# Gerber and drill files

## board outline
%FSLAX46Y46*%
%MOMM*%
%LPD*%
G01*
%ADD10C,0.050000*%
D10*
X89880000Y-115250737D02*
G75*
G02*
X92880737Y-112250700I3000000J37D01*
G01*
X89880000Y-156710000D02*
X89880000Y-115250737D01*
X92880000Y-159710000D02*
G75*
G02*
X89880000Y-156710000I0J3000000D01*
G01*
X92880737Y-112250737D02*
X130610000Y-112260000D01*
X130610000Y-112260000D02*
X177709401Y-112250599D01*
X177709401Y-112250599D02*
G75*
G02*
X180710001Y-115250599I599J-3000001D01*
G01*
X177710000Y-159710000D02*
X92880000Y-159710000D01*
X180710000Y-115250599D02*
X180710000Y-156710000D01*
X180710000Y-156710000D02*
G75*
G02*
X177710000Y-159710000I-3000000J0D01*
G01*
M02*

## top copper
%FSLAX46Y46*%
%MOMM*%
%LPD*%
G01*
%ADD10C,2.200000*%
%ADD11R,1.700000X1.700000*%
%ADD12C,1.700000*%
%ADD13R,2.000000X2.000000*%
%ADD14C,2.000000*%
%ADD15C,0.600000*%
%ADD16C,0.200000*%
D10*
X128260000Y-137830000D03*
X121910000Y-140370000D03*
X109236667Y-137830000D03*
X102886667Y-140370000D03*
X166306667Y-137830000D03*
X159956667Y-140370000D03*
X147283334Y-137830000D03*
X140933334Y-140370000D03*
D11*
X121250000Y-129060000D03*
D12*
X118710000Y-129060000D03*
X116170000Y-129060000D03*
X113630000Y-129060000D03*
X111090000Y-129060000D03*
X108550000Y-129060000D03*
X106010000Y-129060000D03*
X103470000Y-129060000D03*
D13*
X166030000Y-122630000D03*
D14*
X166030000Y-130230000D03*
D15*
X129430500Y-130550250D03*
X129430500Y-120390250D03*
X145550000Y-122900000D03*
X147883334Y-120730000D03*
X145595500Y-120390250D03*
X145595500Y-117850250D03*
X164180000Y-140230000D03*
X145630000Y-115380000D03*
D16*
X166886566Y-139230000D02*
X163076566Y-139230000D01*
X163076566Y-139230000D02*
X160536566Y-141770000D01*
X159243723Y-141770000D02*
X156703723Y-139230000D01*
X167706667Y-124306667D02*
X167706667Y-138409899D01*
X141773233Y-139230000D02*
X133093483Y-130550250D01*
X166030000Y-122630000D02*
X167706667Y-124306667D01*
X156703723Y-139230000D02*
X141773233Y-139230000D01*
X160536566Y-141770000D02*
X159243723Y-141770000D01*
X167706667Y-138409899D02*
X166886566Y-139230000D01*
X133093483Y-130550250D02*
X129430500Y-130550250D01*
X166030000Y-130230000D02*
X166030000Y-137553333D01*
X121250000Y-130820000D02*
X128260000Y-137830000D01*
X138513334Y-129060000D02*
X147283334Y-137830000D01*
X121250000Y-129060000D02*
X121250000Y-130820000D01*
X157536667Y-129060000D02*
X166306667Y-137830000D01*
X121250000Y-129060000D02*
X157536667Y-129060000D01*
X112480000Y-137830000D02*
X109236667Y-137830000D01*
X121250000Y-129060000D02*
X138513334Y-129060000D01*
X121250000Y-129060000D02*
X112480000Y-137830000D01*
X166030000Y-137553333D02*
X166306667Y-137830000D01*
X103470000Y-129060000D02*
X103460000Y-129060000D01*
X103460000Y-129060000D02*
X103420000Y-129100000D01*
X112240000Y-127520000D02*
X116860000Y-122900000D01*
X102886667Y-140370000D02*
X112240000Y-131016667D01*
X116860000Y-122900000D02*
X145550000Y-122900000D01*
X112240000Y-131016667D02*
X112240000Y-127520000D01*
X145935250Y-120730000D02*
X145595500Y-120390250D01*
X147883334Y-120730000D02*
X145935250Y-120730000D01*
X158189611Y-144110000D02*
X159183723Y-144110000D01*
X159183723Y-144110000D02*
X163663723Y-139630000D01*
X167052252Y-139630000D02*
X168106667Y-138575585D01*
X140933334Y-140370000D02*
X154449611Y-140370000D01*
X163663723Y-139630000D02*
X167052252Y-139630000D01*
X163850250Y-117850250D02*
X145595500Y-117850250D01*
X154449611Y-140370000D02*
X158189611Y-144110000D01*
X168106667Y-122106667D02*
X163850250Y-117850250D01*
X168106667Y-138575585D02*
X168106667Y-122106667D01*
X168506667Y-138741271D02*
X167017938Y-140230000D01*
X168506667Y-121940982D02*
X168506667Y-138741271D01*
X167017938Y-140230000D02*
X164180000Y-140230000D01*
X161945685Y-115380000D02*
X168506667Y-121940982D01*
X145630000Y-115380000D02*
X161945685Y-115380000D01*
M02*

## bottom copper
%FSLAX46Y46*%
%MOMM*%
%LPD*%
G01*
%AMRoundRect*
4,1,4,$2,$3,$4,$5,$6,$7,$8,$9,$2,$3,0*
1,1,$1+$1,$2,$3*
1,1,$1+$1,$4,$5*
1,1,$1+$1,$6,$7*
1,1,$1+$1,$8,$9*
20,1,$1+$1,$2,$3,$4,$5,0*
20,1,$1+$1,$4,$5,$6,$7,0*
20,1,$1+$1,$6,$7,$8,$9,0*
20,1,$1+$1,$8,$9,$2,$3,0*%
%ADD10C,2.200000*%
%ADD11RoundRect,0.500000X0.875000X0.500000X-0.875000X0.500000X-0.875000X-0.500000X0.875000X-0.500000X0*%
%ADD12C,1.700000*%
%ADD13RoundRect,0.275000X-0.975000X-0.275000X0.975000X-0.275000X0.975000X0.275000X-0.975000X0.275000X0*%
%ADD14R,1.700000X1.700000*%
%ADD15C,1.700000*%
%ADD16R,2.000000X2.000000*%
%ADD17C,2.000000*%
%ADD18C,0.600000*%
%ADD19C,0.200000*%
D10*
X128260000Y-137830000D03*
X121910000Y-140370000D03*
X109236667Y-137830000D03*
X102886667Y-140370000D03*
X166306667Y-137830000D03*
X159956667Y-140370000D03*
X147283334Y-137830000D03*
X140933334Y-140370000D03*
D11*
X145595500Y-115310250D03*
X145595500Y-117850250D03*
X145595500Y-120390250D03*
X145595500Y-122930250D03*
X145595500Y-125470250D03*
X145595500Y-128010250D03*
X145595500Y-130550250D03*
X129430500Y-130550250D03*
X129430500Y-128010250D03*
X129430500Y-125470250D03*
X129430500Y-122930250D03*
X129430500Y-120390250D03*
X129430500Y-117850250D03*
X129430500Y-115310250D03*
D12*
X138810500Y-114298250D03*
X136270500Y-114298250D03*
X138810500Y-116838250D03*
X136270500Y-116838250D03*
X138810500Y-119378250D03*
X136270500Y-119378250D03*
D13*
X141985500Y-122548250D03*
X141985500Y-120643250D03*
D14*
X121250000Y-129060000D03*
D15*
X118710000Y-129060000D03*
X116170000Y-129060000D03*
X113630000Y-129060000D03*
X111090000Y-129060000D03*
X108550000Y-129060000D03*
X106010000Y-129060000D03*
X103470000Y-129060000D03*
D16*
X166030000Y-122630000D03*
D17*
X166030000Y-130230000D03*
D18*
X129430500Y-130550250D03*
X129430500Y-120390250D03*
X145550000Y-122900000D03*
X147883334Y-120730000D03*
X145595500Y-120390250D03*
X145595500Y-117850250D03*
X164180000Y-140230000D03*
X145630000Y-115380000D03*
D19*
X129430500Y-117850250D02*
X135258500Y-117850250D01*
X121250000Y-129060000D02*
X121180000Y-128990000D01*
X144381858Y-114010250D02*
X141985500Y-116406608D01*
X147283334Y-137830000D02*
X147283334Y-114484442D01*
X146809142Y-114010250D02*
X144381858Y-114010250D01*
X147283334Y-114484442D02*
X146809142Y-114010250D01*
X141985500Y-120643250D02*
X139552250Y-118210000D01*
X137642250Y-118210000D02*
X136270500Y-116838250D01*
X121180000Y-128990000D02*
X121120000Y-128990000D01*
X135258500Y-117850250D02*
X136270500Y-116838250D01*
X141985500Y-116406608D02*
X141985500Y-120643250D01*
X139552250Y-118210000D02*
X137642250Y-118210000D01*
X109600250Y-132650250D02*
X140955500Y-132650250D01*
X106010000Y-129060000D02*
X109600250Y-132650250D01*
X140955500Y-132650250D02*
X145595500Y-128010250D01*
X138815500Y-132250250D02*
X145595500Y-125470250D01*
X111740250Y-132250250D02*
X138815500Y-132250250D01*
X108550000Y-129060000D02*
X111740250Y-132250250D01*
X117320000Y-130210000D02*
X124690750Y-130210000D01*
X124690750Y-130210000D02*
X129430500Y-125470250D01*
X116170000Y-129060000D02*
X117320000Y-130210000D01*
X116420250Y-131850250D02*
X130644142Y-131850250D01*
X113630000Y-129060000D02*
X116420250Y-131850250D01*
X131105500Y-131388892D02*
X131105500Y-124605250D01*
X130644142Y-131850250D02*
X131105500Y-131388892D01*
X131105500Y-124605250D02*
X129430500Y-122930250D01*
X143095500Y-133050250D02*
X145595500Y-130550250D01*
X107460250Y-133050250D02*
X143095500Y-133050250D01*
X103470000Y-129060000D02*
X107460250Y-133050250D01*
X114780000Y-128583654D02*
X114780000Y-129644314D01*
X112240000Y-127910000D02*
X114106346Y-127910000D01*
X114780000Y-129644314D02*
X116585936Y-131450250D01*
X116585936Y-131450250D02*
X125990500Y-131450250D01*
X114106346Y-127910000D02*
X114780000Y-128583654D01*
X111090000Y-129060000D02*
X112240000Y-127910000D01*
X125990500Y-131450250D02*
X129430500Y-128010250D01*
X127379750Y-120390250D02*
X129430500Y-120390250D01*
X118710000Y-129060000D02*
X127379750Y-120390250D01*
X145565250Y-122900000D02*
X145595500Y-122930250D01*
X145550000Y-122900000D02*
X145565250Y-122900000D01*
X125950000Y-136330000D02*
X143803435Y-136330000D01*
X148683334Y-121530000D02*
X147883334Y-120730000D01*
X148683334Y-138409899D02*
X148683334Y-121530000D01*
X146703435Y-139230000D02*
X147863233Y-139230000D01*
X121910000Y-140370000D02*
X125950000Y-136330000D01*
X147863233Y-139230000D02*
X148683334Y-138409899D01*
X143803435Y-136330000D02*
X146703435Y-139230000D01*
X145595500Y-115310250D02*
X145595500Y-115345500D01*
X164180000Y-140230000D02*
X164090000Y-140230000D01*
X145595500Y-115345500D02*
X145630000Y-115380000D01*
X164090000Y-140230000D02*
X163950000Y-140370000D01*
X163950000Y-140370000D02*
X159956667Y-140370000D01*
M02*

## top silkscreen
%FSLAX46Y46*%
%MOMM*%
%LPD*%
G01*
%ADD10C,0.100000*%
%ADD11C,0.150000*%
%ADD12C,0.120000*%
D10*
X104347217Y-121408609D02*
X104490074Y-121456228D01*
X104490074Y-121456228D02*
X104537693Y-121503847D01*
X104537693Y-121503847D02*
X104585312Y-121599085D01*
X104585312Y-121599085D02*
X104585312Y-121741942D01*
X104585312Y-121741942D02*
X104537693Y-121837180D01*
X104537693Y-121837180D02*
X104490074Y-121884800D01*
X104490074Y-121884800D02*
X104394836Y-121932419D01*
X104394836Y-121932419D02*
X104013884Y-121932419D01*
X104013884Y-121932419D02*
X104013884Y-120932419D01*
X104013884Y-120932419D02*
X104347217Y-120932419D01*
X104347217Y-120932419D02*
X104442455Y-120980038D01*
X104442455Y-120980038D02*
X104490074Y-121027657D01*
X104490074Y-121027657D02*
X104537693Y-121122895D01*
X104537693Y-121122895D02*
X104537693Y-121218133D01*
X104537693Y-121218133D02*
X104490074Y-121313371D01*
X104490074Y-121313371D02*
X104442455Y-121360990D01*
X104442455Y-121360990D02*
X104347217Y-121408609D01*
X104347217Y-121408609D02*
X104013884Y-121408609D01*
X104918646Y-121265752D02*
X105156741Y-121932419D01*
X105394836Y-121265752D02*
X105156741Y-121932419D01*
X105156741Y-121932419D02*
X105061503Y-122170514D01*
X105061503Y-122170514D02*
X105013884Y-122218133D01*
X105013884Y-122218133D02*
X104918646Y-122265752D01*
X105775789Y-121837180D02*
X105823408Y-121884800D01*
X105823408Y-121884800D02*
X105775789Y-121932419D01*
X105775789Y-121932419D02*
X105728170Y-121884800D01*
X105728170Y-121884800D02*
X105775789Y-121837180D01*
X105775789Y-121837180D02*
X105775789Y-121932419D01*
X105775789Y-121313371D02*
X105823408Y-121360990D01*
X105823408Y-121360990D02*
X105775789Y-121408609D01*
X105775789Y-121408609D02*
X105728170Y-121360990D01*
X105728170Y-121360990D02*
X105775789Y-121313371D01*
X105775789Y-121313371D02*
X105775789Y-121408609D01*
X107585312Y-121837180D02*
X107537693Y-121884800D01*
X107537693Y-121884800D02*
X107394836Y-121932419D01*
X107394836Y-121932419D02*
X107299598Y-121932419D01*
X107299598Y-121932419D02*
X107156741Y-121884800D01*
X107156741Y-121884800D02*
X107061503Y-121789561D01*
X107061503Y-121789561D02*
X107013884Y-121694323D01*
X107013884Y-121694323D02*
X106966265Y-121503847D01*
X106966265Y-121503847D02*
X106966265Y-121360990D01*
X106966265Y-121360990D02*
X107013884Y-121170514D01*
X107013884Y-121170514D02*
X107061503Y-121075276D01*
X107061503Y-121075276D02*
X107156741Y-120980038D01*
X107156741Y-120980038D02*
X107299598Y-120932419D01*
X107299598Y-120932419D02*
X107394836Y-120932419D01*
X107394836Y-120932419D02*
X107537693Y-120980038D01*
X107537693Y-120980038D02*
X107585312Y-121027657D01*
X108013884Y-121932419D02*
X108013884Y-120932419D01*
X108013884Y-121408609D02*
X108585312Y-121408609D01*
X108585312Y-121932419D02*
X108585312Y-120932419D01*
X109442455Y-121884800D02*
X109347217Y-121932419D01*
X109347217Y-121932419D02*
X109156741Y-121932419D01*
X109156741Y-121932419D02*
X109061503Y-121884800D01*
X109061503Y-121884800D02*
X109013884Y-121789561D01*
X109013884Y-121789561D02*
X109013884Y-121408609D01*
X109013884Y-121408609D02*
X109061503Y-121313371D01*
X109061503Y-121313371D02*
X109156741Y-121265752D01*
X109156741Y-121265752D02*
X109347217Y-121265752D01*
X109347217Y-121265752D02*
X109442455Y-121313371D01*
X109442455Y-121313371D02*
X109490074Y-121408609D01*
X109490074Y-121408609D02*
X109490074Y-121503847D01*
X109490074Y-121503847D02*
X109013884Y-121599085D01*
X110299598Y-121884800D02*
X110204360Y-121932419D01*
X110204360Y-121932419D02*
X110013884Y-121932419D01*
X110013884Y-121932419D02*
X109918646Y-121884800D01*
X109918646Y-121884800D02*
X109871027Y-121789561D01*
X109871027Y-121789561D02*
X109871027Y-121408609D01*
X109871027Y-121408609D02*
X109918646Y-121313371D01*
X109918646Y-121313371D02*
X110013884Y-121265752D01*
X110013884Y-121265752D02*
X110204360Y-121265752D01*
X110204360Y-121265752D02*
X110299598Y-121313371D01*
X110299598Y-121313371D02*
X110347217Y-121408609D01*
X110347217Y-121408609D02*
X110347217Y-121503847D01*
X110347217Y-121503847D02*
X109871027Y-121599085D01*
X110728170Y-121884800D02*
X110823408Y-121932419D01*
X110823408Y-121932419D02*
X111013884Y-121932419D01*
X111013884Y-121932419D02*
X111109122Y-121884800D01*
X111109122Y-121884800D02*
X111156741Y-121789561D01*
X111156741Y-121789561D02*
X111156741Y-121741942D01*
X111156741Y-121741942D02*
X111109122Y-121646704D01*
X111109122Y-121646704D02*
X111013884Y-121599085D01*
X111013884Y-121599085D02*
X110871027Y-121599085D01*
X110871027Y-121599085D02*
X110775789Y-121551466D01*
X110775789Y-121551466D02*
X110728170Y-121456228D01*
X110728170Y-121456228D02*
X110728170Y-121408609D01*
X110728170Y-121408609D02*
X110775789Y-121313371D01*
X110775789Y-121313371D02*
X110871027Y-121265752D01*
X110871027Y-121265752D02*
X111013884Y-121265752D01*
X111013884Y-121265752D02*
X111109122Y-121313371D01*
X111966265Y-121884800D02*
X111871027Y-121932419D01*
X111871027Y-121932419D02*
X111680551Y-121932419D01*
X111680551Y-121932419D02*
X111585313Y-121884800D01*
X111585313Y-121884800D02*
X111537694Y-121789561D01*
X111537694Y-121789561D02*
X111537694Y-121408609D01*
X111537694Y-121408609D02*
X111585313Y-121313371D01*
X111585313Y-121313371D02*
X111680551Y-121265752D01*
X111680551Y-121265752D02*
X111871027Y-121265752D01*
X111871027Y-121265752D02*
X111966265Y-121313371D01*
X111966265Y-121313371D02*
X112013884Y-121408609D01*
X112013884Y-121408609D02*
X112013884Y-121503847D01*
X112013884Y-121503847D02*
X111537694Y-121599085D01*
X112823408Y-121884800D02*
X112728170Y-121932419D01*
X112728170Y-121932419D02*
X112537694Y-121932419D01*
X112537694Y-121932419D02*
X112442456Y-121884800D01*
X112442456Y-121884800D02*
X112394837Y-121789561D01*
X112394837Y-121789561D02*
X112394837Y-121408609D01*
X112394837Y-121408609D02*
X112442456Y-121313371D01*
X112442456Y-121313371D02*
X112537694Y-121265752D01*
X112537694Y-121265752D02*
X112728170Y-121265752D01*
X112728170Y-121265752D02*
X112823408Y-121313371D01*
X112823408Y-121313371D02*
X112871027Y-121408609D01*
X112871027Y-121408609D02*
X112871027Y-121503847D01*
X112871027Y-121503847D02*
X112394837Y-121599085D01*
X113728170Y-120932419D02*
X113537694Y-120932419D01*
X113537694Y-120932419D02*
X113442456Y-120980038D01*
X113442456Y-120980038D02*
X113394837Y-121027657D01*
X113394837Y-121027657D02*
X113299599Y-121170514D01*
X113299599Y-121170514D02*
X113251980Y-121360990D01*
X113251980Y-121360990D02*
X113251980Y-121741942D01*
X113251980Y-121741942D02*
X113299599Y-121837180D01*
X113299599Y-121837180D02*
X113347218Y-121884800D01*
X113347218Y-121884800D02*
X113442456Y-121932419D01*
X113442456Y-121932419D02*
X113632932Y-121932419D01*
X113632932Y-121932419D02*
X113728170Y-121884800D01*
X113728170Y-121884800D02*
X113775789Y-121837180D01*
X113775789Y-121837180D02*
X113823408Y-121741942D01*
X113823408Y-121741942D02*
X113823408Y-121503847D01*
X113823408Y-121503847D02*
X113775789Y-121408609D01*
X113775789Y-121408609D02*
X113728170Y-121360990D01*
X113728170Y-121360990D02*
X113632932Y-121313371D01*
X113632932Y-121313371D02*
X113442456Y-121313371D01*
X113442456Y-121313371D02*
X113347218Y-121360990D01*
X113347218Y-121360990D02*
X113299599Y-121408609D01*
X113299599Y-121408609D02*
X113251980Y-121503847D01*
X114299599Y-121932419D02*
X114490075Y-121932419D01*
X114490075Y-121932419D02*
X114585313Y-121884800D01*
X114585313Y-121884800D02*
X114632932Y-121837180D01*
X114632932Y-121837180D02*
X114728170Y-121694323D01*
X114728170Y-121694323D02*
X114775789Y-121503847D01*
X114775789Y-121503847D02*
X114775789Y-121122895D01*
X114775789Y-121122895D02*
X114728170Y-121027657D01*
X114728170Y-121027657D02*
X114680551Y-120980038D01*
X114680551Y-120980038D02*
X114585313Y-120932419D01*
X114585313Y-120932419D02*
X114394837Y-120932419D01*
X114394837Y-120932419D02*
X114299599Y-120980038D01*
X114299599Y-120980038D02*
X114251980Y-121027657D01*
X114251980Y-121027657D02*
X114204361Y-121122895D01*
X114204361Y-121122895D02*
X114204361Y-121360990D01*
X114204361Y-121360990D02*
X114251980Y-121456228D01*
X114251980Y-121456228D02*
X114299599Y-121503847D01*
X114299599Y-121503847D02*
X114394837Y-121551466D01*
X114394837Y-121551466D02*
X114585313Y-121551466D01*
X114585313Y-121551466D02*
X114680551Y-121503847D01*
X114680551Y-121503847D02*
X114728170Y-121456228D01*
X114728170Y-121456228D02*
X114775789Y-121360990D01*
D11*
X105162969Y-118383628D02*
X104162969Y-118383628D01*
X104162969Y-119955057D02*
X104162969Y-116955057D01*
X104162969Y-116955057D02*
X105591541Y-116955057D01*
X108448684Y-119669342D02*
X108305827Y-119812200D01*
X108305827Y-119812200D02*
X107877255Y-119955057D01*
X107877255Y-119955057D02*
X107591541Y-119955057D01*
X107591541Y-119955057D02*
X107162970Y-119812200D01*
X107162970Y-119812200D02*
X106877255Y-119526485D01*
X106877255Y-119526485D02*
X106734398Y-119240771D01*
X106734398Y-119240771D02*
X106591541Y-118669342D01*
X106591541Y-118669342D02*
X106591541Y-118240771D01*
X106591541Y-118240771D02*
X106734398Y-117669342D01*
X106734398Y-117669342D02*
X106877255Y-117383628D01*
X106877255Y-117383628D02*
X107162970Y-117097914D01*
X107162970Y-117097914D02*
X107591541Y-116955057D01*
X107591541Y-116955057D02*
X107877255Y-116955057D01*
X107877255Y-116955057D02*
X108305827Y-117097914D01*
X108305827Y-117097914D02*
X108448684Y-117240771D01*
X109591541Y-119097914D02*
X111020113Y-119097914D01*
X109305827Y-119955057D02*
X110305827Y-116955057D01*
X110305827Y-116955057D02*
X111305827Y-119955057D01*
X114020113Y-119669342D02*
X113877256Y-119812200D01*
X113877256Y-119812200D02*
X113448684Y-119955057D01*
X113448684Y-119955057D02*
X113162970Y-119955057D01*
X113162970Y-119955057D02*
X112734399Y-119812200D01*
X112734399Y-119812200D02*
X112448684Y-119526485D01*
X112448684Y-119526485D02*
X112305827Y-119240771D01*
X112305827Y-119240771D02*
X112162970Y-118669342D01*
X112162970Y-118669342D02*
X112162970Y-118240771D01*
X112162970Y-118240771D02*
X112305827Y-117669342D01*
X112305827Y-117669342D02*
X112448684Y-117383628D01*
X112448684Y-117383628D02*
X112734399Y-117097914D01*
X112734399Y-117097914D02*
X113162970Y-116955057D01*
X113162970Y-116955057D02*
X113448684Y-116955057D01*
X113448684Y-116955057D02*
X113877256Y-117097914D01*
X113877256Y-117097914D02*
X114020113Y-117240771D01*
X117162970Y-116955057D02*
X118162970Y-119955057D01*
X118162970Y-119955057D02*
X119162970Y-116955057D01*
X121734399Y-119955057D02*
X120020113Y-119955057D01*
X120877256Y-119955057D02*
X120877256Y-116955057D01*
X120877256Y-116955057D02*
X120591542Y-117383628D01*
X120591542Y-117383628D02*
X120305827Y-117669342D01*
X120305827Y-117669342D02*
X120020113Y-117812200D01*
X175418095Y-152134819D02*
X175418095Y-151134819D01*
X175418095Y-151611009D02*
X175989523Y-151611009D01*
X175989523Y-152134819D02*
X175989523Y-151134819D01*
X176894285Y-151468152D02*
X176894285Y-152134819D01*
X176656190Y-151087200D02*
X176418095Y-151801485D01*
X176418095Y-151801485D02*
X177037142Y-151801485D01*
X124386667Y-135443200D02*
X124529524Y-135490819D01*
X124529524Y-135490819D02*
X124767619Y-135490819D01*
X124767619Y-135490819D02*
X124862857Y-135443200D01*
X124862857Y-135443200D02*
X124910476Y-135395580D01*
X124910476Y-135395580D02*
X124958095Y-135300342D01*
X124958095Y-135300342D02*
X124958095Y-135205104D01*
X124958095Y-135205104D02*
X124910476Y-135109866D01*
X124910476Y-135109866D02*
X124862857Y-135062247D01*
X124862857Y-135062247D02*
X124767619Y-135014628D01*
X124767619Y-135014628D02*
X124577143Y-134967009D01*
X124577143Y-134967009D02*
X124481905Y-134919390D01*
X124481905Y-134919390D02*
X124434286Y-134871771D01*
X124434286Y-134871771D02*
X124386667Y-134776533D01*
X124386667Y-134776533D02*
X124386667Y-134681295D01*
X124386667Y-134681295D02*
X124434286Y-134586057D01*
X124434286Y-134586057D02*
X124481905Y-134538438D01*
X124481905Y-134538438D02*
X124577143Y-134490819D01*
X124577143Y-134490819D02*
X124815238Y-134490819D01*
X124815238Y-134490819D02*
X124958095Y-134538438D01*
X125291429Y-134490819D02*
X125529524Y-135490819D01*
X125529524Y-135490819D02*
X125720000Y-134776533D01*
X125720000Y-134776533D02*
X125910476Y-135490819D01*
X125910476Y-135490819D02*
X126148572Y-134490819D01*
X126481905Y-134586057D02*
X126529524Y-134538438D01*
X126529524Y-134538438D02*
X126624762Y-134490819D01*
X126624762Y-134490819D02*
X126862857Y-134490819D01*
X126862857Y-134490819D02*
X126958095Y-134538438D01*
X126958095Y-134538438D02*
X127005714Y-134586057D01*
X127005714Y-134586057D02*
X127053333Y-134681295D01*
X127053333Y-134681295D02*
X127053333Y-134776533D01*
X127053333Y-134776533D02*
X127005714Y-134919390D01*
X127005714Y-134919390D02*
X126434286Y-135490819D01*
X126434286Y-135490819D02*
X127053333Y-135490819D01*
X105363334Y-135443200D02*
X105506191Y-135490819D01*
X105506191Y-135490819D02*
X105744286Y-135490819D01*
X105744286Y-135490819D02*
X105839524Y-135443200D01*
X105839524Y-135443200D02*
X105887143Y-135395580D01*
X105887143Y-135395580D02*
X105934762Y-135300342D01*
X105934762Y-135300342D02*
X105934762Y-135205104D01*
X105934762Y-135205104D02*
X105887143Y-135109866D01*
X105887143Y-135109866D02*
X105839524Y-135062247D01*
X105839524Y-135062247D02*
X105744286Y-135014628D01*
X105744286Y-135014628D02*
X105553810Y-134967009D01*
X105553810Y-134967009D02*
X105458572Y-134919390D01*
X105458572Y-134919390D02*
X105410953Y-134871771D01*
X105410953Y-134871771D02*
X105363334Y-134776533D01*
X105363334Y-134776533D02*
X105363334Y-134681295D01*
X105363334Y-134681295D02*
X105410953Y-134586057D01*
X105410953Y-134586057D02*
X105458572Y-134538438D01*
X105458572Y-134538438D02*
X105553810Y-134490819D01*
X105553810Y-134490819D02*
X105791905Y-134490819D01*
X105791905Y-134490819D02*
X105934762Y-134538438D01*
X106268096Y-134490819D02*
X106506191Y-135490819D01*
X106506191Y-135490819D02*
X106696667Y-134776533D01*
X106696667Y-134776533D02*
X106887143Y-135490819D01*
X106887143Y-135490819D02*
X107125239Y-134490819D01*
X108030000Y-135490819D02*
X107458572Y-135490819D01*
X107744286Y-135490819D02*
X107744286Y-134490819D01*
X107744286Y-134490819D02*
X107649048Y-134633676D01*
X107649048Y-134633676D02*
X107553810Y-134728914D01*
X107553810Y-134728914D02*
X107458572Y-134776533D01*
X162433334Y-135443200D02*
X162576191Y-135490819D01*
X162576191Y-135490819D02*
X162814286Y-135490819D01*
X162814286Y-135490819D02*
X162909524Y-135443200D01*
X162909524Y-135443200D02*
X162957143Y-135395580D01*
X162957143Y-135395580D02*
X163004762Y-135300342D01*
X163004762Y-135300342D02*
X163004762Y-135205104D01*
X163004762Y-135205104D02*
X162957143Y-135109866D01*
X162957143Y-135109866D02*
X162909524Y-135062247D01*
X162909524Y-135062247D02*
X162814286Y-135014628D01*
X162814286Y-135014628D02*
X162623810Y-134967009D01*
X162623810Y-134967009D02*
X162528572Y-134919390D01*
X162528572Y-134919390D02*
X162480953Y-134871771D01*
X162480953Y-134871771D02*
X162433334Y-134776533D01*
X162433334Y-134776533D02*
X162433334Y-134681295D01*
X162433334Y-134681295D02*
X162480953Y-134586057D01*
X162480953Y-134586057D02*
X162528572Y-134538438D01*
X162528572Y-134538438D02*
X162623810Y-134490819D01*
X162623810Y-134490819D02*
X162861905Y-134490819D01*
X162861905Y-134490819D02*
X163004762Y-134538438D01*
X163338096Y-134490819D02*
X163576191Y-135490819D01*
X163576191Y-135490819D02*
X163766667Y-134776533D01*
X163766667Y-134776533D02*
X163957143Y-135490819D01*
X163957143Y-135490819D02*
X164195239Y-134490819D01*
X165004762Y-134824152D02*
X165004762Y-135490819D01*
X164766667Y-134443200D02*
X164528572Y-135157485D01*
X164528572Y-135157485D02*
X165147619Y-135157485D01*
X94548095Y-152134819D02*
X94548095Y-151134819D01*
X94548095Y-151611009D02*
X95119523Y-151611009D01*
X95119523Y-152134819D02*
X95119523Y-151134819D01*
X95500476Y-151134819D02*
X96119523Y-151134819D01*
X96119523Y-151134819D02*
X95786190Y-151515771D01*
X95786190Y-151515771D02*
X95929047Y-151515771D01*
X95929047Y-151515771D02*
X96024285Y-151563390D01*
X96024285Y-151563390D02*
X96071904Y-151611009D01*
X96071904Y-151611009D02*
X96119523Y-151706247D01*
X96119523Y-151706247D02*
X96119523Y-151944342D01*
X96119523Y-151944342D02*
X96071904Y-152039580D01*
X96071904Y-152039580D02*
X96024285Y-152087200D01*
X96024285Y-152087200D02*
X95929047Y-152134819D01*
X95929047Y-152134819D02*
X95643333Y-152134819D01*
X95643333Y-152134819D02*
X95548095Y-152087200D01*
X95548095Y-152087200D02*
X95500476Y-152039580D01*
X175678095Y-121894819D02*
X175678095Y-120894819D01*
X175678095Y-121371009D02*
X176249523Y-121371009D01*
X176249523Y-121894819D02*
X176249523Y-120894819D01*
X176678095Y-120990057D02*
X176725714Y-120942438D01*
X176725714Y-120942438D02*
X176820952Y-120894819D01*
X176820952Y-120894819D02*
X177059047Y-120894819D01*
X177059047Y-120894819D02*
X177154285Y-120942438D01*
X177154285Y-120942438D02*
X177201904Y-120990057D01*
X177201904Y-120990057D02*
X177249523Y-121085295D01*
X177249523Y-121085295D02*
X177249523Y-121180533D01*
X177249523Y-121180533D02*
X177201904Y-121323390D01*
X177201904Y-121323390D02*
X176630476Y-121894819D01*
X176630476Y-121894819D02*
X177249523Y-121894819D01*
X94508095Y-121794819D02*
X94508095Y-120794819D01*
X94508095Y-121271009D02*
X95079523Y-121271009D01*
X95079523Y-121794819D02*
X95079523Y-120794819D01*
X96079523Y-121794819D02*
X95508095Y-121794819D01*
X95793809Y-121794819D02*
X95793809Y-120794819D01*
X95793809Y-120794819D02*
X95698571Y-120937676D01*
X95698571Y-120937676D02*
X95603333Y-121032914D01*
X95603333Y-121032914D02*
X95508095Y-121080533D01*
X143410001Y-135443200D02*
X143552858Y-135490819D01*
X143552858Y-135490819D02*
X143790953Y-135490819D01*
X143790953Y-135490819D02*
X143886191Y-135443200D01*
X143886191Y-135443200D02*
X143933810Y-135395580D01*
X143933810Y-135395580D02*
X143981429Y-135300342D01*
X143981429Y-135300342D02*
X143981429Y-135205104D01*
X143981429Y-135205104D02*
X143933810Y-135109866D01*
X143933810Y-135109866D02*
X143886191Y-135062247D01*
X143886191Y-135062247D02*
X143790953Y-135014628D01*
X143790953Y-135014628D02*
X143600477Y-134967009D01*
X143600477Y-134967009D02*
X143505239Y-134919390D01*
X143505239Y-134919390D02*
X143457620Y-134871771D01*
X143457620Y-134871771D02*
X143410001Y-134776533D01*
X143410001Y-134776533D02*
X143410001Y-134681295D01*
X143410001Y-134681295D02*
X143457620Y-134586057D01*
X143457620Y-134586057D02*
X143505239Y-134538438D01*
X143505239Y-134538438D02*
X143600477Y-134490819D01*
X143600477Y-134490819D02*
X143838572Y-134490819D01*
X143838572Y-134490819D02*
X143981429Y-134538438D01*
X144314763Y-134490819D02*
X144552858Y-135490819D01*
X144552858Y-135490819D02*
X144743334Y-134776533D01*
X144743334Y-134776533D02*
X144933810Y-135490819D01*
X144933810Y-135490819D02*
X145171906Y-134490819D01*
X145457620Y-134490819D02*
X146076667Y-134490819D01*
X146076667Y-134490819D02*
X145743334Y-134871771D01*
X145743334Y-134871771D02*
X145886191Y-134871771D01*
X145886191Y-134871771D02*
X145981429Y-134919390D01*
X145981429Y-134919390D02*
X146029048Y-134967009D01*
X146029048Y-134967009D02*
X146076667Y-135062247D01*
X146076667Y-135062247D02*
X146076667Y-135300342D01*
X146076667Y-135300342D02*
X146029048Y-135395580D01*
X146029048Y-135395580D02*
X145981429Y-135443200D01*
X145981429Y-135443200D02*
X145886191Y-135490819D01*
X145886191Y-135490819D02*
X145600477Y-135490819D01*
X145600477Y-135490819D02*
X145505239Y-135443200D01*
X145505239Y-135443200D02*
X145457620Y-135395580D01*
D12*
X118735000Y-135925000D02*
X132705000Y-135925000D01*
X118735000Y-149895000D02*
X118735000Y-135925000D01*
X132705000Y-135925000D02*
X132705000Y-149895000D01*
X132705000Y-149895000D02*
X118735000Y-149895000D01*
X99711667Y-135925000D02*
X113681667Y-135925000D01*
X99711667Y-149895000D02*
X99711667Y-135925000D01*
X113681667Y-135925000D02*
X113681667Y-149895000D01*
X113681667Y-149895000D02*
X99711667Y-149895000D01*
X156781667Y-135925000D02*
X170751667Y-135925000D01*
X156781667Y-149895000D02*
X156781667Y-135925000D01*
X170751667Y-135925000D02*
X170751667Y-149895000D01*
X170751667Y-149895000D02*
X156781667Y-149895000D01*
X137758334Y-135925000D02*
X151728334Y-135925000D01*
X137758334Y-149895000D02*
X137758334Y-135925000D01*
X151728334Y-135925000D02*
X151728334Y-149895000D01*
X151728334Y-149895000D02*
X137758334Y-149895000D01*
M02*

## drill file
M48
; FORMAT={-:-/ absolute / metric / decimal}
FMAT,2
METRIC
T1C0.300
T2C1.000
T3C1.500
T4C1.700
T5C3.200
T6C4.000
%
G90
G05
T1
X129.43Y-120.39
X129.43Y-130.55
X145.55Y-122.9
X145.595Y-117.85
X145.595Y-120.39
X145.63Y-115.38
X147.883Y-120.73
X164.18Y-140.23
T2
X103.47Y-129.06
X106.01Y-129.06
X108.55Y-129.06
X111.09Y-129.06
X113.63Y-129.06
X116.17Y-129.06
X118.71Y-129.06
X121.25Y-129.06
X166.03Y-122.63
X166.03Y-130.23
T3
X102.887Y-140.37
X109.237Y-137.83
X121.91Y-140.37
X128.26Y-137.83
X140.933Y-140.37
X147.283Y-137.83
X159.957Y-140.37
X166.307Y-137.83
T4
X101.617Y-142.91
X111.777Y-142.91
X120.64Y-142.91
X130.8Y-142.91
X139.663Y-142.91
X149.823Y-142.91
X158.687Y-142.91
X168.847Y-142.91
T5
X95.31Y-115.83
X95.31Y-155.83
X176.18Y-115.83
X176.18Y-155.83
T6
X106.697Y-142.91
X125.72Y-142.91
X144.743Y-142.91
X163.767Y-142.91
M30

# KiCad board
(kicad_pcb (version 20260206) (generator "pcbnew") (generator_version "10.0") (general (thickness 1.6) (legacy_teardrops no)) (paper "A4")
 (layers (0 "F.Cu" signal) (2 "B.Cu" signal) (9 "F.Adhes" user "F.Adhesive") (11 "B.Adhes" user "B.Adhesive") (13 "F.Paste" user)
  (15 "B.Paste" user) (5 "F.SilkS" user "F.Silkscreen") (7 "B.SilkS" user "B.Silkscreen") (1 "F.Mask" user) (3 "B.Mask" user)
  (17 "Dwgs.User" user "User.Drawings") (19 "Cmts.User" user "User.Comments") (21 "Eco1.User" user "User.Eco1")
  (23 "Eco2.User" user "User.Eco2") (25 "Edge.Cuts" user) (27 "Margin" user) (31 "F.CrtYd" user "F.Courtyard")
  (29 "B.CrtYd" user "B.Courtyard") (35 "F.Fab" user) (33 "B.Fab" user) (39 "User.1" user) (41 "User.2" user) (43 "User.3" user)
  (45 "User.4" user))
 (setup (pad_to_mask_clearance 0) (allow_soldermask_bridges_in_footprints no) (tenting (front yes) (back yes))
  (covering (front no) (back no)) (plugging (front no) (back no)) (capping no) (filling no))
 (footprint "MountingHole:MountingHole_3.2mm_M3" (layer "F.Cu") (at 176.18 155.83)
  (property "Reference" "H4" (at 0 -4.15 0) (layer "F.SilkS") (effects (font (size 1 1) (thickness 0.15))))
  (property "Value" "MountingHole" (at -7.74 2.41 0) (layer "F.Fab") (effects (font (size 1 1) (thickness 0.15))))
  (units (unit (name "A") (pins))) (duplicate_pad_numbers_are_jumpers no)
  (pad "" np_thru_hole circle (at 0 0) (size 3.2 3.2) (drill 3.2) (layers "*.Cu" "*.Mask")))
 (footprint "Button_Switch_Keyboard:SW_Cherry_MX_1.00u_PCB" (layer "F.Cu") (at 128.26 137.83)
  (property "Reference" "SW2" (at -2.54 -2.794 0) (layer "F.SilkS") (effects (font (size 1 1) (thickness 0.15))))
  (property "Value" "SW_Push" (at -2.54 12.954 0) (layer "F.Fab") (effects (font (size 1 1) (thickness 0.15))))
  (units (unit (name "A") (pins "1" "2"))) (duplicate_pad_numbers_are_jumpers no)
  (fp_line (start -9.525 -1.905) (end 4.445 -1.905) (stroke (width 0.12) (type solid)) (layer "F.SilkS"))
  (fp_line (start -9.525 12.065) (end -9.525 -1.905) (stroke (width 0.12) (type solid)) (layer "F.SilkS"))
  (fp_line (start 4.445 -1.905) (end 4.445 12.065) (stroke (width 0.12) (type solid)) (layer "F.SilkS"))
  (fp_line (start 4.445 12.065) (end -9.525 12.065) (stroke (width 0.12) (type solid)) (layer "F.SilkS"))
  (pad "" np_thru_hole circle (at -7.62 5.08) (size 1.7 1.7) (drill 1.7) (layers "*.Cu" "*.Mask"))
  (pad "" np_thru_hole circle (at -2.54 5.08) (size 4 4) (drill 4) (layers "*.Cu" "*.Mask"))
  (pad "" np_thru_hole circle (at 2.54 5.08) (size 1.7 1.7) (drill 1.7) (layers "*.Cu" "*.Mask"))
  (pad "1" thru_hole circle (at 0 0) (size 2.2 2.2) (drill 1.5) (layers "*.Cu" "*.Mask") (remove_unused_layers no) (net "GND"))
  (pad "2" thru_hole circle (at -6.35 2.54) (size 2.2 2.2) (drill 1.5) (layers "*.Cu" "*.Mask") (remove_unused_layers no)
   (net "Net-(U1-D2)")))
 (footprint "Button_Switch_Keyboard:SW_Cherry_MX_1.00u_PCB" (layer "F.Cu") (at 109.236667 137.83)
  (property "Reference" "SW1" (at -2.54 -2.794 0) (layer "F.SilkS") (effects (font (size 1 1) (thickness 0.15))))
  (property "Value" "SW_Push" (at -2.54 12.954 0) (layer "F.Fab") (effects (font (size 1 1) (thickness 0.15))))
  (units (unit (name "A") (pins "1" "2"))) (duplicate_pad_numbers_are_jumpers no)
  (fp_line (start -9.525 -1.905) (end 4.445 -1.905) (stroke (width 0.12) (type solid)) (layer "F.SilkS"))
  (fp_line (start -9.525 12.065) (end -9.525 -1.905) (stroke (width 0.12) (type solid)) (layer "F.SilkS"))
  (fp_line (start 4.445 -1.905) (end 4.445 12.065) (stroke (width 0.12) (type solid)) (layer "F.SilkS"))
  (fp_line (start 4.445 12.065) (end -9.525 12.065) (stroke (width 0.12) (type solid)) (layer "F.SilkS"))
  (pad "" np_thru_hole circle (at -7.62 5.08) (size 1.7 1.7) (drill 1.7) (layers "*.Cu" "*.Mask"))
  (pad "" np_thru_hole circle (at -2.54 5.08) (size 4 4) (drill 4) (layers "*.Cu" "*.Mask"))
  (pad "" np_thru_hole circle (at 2.54 5.08) (size 1.7 1.7) (drill 1.7) (layers "*.Cu" "*.Mask"))
  (pad "1" thru_hole circle (at 0 0) (size 2.2 2.2) (drill 1.5) (layers "*.Cu" "*.Mask") (remove_unused_layers no) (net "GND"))
  (pad "2" thru_hole circle (at -6.35 2.54) (size 2.2 2.2) (drill 1.5) (layers "*.Cu" "*.Mask") (remove_unused_layers no)
   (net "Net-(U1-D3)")))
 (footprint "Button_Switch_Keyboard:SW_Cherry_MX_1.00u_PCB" (layer "F.Cu") (at 166.306667 137.83)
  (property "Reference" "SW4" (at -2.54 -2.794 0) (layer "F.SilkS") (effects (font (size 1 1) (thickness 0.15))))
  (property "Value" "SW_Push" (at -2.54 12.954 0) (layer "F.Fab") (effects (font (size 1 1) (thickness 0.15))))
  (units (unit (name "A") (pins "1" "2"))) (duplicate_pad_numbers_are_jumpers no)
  (fp_line (start -9.525 -1.905) (end 4.445 -1.905) (stroke (width 0.12) (type solid)) (layer "F.SilkS"))
  (fp_line (start -9.525 12.065) (end -9.525 -1.905) (stroke (width 0.12) (type solid)) (layer "F.SilkS"))
  (fp_line (start 4.445 -1.905) (end 4.445 12.065) (stroke (width 0.12) (type solid)) (layer "F.SilkS"))
  (fp_line (start 4.445 12.065) (end -9.525 12.065) (stroke (width 0.12) (type solid)) (layer "F.SilkS"))
  (pad "" np_thru_hole circle (at -7.62 5.08) (size 1.7 1.7) (drill 1.7) (layers "*.Cu" "*.Mask"))
  (pad "" np_thru_hole circle (at -2.54 5.08) (size 4 4) (drill 4) (layers "*.Cu" "*.Mask"))
  (pad "" np_thru_hole circle (at 2.54 5.08) (size 1.7 1.7) (drill 1.7) (layers "*.Cu" "*.Mask"))
  (pad "1" thru_hole circle (at 0 0) (size 2.2 2.2) (drill 1.5) (layers "*.Cu" "*.Mask") (remove_unused_layers no) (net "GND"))
  (pad "2" thru_hole circle (at -6.35 2.54) (size 2.2 2.2) (drill 1.5) (layers "*.Cu" "*.Mask") (remove_unused_layers no)
   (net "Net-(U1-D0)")))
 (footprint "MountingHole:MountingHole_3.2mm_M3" (layer "F.Cu") (at 95.31 155.83)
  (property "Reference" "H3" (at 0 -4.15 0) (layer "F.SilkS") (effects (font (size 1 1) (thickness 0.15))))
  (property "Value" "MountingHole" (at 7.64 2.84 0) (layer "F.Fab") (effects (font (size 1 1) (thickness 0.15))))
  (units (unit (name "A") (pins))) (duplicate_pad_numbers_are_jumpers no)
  (pad "" np_thru_hole circle (at 0 0) (size 3.2 3.2) (drill 3.2) (layers "*.Cu" "*.Mask")))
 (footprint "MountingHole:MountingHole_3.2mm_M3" (layer "F.Cu") (at 176.18 115.83)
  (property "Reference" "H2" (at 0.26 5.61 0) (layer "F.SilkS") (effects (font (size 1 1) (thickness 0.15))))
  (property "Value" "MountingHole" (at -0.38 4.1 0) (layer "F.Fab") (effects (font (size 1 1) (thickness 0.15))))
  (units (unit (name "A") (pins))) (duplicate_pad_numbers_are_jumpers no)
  (pad "" np_thru_hole circle (at 0 0) (size 3.2 3.2) (drill 3.2) (layers "*.Cu" "*.Mask")))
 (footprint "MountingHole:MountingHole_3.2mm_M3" (layer "F.Cu") (at 95.31 115.83)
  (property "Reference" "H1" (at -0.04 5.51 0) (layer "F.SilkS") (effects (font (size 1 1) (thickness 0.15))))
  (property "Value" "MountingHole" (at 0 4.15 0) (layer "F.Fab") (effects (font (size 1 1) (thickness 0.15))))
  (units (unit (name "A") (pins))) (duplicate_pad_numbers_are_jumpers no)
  (pad "" np_thru_hole circle (at 0 0) (size 3.2 3.2) (drill 3.2) (layers "*.Cu" "*.Mask")))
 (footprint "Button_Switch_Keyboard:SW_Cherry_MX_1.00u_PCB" (layer "F.Cu") (at 147.283334 137.83)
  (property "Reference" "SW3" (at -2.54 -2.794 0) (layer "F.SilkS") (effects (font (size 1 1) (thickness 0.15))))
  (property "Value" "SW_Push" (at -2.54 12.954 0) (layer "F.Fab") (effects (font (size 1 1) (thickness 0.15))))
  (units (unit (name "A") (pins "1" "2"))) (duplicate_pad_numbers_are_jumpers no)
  (fp_line (start -9.525 -1.905) (end 4.445 -1.905) (stroke (width 0.12) (type solid)) (layer "F.SilkS"))
  (fp_line (start -9.525 12.065) (end -9.525 -1.905) (stroke (width 0.12) (type solid)) (layer "F.SilkS"))
  (fp_line (start 4.445 -1.905) (end 4.445 12.065) (stroke (width 0.12) (type solid)) (layer "F.SilkS"))
  (fp_line (start 4.445 12.065) (end -9.525 12.065) (stroke (width 0.12) (type solid)) (layer "F.SilkS"))
  (pad "" np_thru_hole circle (at -7.62 5.08) (size 1.7 1.7) (drill 1.7) (layers "*.Cu" "*.Mask"))
  (pad "" np_thru_hole circle (at -2.54 5.08) (size 4 4) (drill 4) (layers "*.Cu" "*.Mask"))
  (pad "" np_thru_hole circle (at 2.54 5.08) (size 1.7 1.7) (drill 1.7) (layers "*.Cu" "*.Mask"))
  (pad "1" thru_hole circle (at 0 0) (size 2.2 2.2) (drill 1.5) (layers "*.Cu" "*.Mask") (remove_unused_layers no) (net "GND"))
  (pad "2" thru_hole circle (at -6.35 2.54) (size 2.2 2.2) (drill 1.5) (layers "*.Cu" "*.Mask") (remove_unused_layers no)
   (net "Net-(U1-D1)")))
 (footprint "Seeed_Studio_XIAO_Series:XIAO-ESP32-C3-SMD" (layer "B.Cu") (at 146.4305 133.43025 180)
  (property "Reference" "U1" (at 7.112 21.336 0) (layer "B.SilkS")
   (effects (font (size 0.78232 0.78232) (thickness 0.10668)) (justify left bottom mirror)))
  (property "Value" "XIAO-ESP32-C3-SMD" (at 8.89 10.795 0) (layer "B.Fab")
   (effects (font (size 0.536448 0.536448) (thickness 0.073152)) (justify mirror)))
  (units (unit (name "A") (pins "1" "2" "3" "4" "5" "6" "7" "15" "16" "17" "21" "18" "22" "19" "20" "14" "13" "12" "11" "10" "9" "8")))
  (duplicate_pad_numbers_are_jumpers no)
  (pad "1" smd roundrect (at 0.835 18.12 180) (size 2.75 2) (layers "B.Cu" "B.Mask" "B.Paste") (roundrect_rratio 0.25) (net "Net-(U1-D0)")
   (solder_mask_margin 0.0508) (thermal_bridge_angle 45))
  (pad "2" smd roundrect (at 0.835 15.58 180) (size 2.75 2) (layers "B.Cu" "B.Mask" "B.Paste") (roundrect_rratio 0.25) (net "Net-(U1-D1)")
   (solder_mask_margin 0.0508) (thermal_bridge_angle 45))
  (pad "3" smd roundrect (at 0.835 13.04 180) (size 2.75 2) (layers "B.Cu" "B.Mask" "B.Paste") (roundrect_rratio 0.25) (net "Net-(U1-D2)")
   (solder_mask_margin 0.0508) (thermal_bridge_angle 45))
  (pad "4" smd roundrect (at 0.835 10.5 180) (size 2.75 2) (layers "B.Cu" "B.Mask" "B.Paste") (roundrect_rratio 0.25) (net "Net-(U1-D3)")
   (solder_mask_margin 0.0508) (thermal_bridge_angle 45))
  (pad "5" smd roundrect (at 0.835 7.96 180) (size 2.75 2) (layers "B.Cu" "B.Mask" "B.Paste") (roundrect_rratio 0.25) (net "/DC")
   (solder_mask_margin 0.0508) (thermal_bridge_angle 45))
  (pad "6" smd roundrect (at 0.835 5.42 180) (size 2.75 2) (layers "B.Cu" "B.Mask" "B.Paste") (roundrect_rratio 0.25) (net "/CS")
   (solder_mask_margin 0.0508) (thermal_bridge_angle 45))
  (pad "7" smd roundrect (at 0.835 2.88 180) (size 2.75 2) (layers "B.Cu" "B.Mask" "B.Paste") (roundrect_rratio 0.25) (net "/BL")
   (solder_mask_margin 0.0508) (thermal_bridge_angle 45))
  (pad "8" smd roundrect (at 17 2.88 180) (size 2.75 2) (layers "B.Cu" "B.Mask" "B.Paste") (roundrect_rratio 0.25) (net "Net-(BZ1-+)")
   (solder_mask_margin 0.0508) (thermal_bridge_angle 45))
  (pad "9" smd roundrect (at 17 5.42 180) (size 2.75 2) (layers "B.Cu" "B.Mask" "B.Paste") (roundrect_rratio 0.25) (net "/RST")
   (solder_mask_margin 0.0508) (thermal_bridge_angle 45))
  (pad "10" smd roundrect (at 17 7.96 180) (size 2.75 2) (layers "B.Cu" "B.Mask" "B.Paste") (roundrect_rratio 0.25) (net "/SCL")
   (solder_mask_margin 0.0508) (thermal_bridge_angle 45))
  (pad "11" smd roundrect (at 17 10.5 180) (size 2.75 2) (layers "B.Cu" "B.Mask" "B.Paste") (roundrect_rratio 0.25) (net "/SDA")
   (solder_mask_margin 0.0508) (thermal_bridge_angle 45))
  (pad "12" smd roundrect (at 17 13.04 180) (size 2.75 2) (layers "B.Cu" "B.Mask" "B.Paste") (roundrect_rratio 0.25) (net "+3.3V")
   (solder_mask_margin 0.0508) (thermal_bridge_angle 45))
  (pad "13" smd roundrect (at 17 15.58 180) (size 2.75 2) (layers "B.Cu" "B.Mask" "B.Paste") (roundrect_rratio 0.25) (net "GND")
   (solder_mask_margin 0.0508) (thermal_bridge_angle 45))
  (pad "14" smd roundrect (at 17 18.12 180) (size 2.75 2) (layers "B.Cu" "B.Mask" "B.Paste") (roundrect_rratio 0.25)
   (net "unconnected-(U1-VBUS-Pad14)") (solder_mask_margin 0.0508) (thermal_bridge_angle 45))
  (pad "15" smd circle (at 7.62 19.132 180) (size 1.7 1.7) (layers "B.Cu" "B.Mask" "B.Paste") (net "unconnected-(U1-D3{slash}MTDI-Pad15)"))
  (pad "16" smd circle (at 10.16 19.132 180) (size 1.7 1.7) (layers "B.Cu" "B.Mask" "B.Paste") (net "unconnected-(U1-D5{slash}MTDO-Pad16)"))
  (pad "17" smd circle (at 7.62 16.592 180) (size 1.7 1.7) (layers "B.Cu" "B.Mask" "B.Paste") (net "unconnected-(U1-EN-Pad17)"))
  (pad "18" smd circle (at 10.16 16.592 180) (size 1.7 1.7) (layers "B.Cu" "B.Mask" "B.Paste") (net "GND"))
  (pad "19" smd circle (at 7.62 14.052 180) (size 1.7 1.7) (layers "B.Cu" "B.Mask" "B.Paste") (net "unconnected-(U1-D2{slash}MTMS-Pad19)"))
  (pad "20" smd circle (at 10.16 14.052 180) (size 1.7 1.7) (layers "B.Cu" "B.Mask" "B.Paste") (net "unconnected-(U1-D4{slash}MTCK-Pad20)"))
  (pad "21" smd roundrect (at 4.445 10.882) (size 2.5 1.1) (layers "B.Cu" "B.Mask" "B.Paste") (roundrect_rratio 0.25)
   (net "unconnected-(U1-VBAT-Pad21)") (thermal_bridge_angle 45))
  (pad "22" smd roundrect (at 4.445 12.787) (size 2.5 1.1) (layers "B.Cu" "B.Mask" "B.Paste") (roundrect_rratio 0.25) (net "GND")
   (thermal_bridge_angle 45)))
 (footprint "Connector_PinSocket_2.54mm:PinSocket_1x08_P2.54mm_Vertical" (layer "B.Cu") (at 121.25 129.06 90)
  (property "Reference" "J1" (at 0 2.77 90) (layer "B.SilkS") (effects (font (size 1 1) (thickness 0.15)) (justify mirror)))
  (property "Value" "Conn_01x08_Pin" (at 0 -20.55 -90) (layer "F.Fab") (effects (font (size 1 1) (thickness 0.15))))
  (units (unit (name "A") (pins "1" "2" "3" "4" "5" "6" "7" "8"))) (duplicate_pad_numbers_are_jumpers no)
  (pad "1" thru_hole rect (at 0 0 90) (size 1.7 1.7) (drill 1) (layers "*.Cu" "*.Mask") (remove_unused_layers no) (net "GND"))
  (pad "2" thru_hole circle (at 0 -2.54 90) (size 1.7 1.7) (drill 1) (layers "*.Cu" "*.Mask") (remove_unused_layers no) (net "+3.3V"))
  (pad "3" thru_hole circle (at 0 -5.08 90) (size 1.7 1.7) (drill 1) (layers "*.Cu" "*.Mask") (remove_unused_layers no) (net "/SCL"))
  (pad "4" thru_hole circle (at 0 -7.62 90) (size 1.7 1.7) (drill 1) (layers "*.Cu" "*.Mask") (remove_unused_layers no) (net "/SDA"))
  (pad "5" thru_hole circle (at 0 -10.16 90) (size 1.7 1.7) (drill 1) (layers "*.Cu" "*.Mask") (remove_unused_layers no) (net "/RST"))
  (pad "6" thru_hole circle (at 0 -12.7 90) (size 1.7 1.7) (drill 1) (layers "*.Cu" "*.Mask") (remove_unused_layers no) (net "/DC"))
  (pad "7" thru_hole circle (at 0 -15.24 90) (size 1.7 1.7) (drill 1) (layers "*.Cu" "*.Mask") (remove_unused_layers no) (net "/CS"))
  (pad "8" thru_hole circle (at 0 -17.78 90) (size 1.7 1.7) (drill 1) (layers "*.Cu" "*.Mask") (remove_unused_layers no) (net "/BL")))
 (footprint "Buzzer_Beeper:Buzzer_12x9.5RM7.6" (layer "B.Cu") (at 166.03 122.63 -90)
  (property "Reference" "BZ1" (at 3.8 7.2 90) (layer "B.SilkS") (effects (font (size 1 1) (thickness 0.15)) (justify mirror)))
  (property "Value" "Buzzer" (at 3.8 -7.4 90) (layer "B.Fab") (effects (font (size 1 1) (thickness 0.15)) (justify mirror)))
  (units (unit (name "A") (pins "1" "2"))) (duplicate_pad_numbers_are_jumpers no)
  (pad "1" thru_hole rect (at 0 0 270) (size 2 2) (drill 1) (layers "*.Cu" "*.Mask") (remove_unused_layers no) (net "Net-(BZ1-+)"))
  (pad "2" thru_hole circle (at 7.6 0 270) (size 2 2) (drill 1) (layers "*.Cu" "*.Mask") (remove_unused_layers no) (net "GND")))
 (gr_arc (start 89.88 115.250737) (mid 90.75894 113.129156) (end 92.880737 112.250737) (stroke (width 0.05) (type default))
  (layer "Edge.Cuts"))
 (gr_line (start 89.88 156.71) (end 89.88 115.250737) (stroke (width 0.05) (type default)) (layer "Edge.Cuts"))
 (gr_arc (start 92.88 159.71) (mid 90.75868 158.83132) (end 89.88 156.71) (stroke (width 0.05) (type default)) (layer "Edge.Cuts"))
 (gr_line (start 92.880737 112.250737) (end 130.61 112.26) (stroke (width 0.05) (type default)) (layer "Edge.Cuts"))
 (gr_line (start 130.61 112.26) (end 177.709401 112.250599) (stroke (width 0.05) (type default)) (layer "Edge.Cuts"))
 (gr_arc (start 177.709401 112.250599) (mid 179.831109 113.129067) (end 180.71 115.250599) (stroke (width 0.05) (type default))
  (layer "Edge.Cuts"))
 (gr_line (start 177.71 159.71) (end 92.88 159.71) (stroke (width 0.05) (type default)) (layer "Edge.Cuts"))
 (gr_line (start 180.71 115.250599) (end 180.71 156.71) (stroke (width 0.05) (type default)) (layer "Edge.Cuts"))
 (gr_arc (start 180.71 156.71) (mid 179.83132 158.83132) (end 177.71 159.71) (stroke (width 0.05) (type default)) (layer "Edge.Cuts"))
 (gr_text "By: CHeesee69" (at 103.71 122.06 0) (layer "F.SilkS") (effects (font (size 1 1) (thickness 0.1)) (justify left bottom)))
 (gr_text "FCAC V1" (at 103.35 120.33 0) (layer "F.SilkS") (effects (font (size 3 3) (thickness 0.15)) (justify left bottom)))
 (segment (start 166.886566 139.23) (end 163.076566 139.23) (width 0.2) (layer "F.Cu") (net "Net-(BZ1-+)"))
 (segment (start 163.076566 139.23) (end 160.536566 141.77) (width 0.2) (layer "F.Cu") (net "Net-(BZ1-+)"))
 (segment (start 159.243723 141.77) (end 156.703723 139.23) (width 0.2) (layer "F.Cu") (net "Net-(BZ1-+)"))
 (segment (start 167.706667 124.306667) (end 167.706667 138.409899) (width 0.2) (layer "F.Cu") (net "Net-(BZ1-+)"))
 (segment (start 141.773233 139.23) (end 133.093483 130.55025) (width 0.2) (layer "F.Cu") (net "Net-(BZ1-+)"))
 (segment (start 166.03 122.63) (end 167.706667 124.306667) (width 0.2) (layer "F.Cu") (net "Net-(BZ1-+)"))
 (segment (start 156.703723 139.23) (end 141.773233 139.23) (width 0.2) (layer "F.Cu") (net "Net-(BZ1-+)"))
 (segment (start 160.536566 141.77) (end 159.243723 141.77) (width 0.2) (layer "F.Cu") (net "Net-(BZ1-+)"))
 (segment (start 167.706667 138.409899) (end 166.886566 139.23) (width 0.2) (layer "F.Cu") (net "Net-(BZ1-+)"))
 (segment (start 133.093483 130.55025) (end 129.4305 130.55025) (width 0.2) (layer "F.Cu") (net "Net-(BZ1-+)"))
 (via (at 129.4305 130.55025) (size 0.6) (drill 0.3) (layers "F.Cu" "B.Cu") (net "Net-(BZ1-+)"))
 (segment (start 166.03 130.23) (end 166.03 137.553333) (width 0.2) (layer "F.Cu") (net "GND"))
 (segment (start 121.25 130.82) (end 128.26 137.83) (width 0.2) (layer "F.Cu") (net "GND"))
 (segment (start 138.513334 129.06) (end 147.283334 137.83) (width 0.2) (layer "F.Cu") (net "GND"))
 (segment (start 121.25 129.06) (end 121.25 130.82) (width 0.2) (layer "F.Cu") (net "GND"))
 (segment (start 157.536667 129.06) (end 166.306667 137.83) (width 0.2) (layer "F.Cu") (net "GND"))
 (segment (start 121.25 129.06) (end 157.536667 129.06) (width 0.2) (layer "F.Cu") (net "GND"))
 (segment (start 112.48 137.83) (end 109.236667 137.83) (width 0.2) (layer "F.Cu") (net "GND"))
 (segment (start 121.25 129.06) (end 138.513334 129.06) (width 0.2) (layer "F.Cu") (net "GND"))
 (segment (start 121.25 129.06) (end 112.48 137.83) (width 0.2) (layer "F.Cu") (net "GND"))
 (segment (start 166.03 137.553333) (end 166.306667 137.83) (width 0.2) (layer "F.Cu") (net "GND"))
 (segment (start 129.4305 117.85025) (end 135.2585 117.85025) (width 0.2) (layer "B.Cu") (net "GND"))
 (segment (start 121.25 129.06) (end 121.18 128.99) (width 0.2) (layer "B.Cu") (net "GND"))
 (segment (start 144.381858 114.01025) (end 141.9855 116.406608) (width 0.2) (layer "B.Cu") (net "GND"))
 (segment (start 147.283334 137.83) (end 147.283334 114.484442) (width 0.2) (layer "B.Cu") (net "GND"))
 (segment (start 146.809142 114.01025) (end 144.381858 114.01025) (width 0.2) (layer "B.Cu") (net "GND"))
 (segment (start 147.283334 114.484442) (end 146.809142 114.01025) (width 0.2) (layer "B.Cu") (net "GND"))
 (segment (start 141.9855 120.64325) (end 139.55225 118.21) (width 0.2) (layer "B.Cu") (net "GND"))
 (segment (start 137.64225 118.21) (end 136.2705 116.83825) (width 0.2) (layer "B.Cu") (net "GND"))
 (segment (start 121.18 128.99) (end 121.12 128.99) (width 0.2) (layer "B.Cu") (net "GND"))
 (segment (start 135.2585 117.85025) (end 136.2705 116.83825) (width 0.2) (layer "B.Cu") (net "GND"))
 (segment (start 141.9855 116.406608) (end 141.9855 120.64325) (width 0.2) (layer "B.Cu") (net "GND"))
 (segment (start 139.55225 118.21) (end 137.64225 118.21) (width 0.2) (layer "B.Cu") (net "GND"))
 (segment (start 109.60025 132.65025) (end 140.9555 132.65025) (width 0.2) (layer "B.Cu") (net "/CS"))
 (segment (start 106.01 129.06) (end 109.60025 132.65025) (width 0.2) (layer "B.Cu") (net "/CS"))
 (segment (start 140.9555 132.65025) (end 145.5955 128.01025) (width 0.2) (layer "B.Cu") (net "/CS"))
 (segment (start 138.8155 132.25025) (end 145.5955 125.47025) (width 0.2) (layer "B.Cu") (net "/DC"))
 (segment (start 111.74025 132.25025) (end 138.8155 132.25025) (width 0.2) (layer "B.Cu") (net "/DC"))
 (segment (start 108.55 129.06) (end 111.74025 132.25025) (width 0.2) (layer "B.Cu") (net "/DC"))
 (segment (start 117.32 130.21) (end 124.69075 130.21) (width 0.2) (layer "B.Cu") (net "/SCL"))
 (segment (start 124.69075 130.21) (end 129.4305 125.47025) (width 0.2) (layer "B.Cu") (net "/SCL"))
 (segment (start 116.17 129.06) (end 117.32 130.21) (width 0.2) (layer "B.Cu") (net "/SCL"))
 (segment (start 116.42025 131.85025) (end 130.644142 131.85025) (width 0.2) (layer "B.Cu") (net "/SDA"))
 (segment (start 113.63 129.06) (end 116.42025 131.85025) (width 0.2) (layer "B.Cu") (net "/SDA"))
 (segment (start 131.1055 131.388892) (end 131.1055 124.60525) (width 0.2) (layer "B.Cu") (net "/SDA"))
 (segment (start 130.644142 131.85025) (end 131.1055 131.388892) (width 0.2) (layer "B.Cu") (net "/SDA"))
 (segment (start 131.1055 124.60525) (end 129.4305 122.93025) (width 0.2) (layer "B.Cu") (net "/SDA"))
 (segment (start 103.47 129.06) (end 103.46 129.06) (width 0.2) (layer "F.Cu") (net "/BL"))
 (segment (start 103.46 129.06) (end 103.42 129.1) (width 0.2) (layer "F.Cu") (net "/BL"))
 (segment (start 143.0955 133.05025) (end 145.5955 130.55025) (width 0.2) (layer "B.Cu") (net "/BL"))
 (segment (start 107.46025 133.05025) (end 143.0955 133.05025) (width 0.2) (layer "B.Cu") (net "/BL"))
 (segment (start 103.47 129.06) (end 107.46025 133.05025) (width 0.2) (layer "B.Cu") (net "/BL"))
 (segment (start 114.78 128.583654) (end 114.78 129.644314) (width 0.2) (layer "B.Cu") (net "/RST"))
 (segment (start 112.24 127.91) (end 114.106346 127.91) (width 0.2) (layer "B.Cu") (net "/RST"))
 (segment (start 114.78 129.644314) (end 116.585936 131.45025) (width 0.2) (layer "B.Cu") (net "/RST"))
 (segment (start 116.585936 131.45025) (end 125.9905 131.45025) (width 0.2) (layer "B.Cu") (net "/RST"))
 (segment (start 114.106346 127.91) (end 114.78 128.583654) (width 0.2) (layer "B.Cu") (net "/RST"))
 (segment (start 111.09 129.06) (end 112.24 127.91) (width 0.2) (layer "B.Cu") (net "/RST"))
 (segment (start 125.9905 131.45025) (end 129.4305 128.01025) (width 0.2) (layer "B.Cu") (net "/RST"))
 (via (at 129.4305 120.39025) (size 0.6) (drill 0.3) (layers "F.Cu" "B.Cu") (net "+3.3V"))
 (segment (start 127.37975 120.39025) (end 129.4305 120.39025) (width 0.2) (layer "B.Cu") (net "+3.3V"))
 (segment (start 118.71 129.06) (end 127.37975 120.39025) (width 0.2) (layer "B.Cu") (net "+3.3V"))
 (segment (start 112.24 127.52) (end 116.86 122.9) (width 0.2) (layer "F.Cu") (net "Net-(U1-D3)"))
 (segment (start 102.886667 140.37) (end 112.24 131.016667) (width 0.2) (layer "F.Cu") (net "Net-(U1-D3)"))
 (segment (start 116.86 122.9) (end 145.55 122.9) (width 0.2) (layer "F.Cu") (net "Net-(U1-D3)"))
 (segment (start 112.24 131.016667) (end 112.24 127.52) (width 0.2) (layer "F.Cu") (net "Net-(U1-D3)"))
 (via (at 145.55 122.9) (size 0.6) (drill 0.3) (layers "F.Cu" "B.Cu") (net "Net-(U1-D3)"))
 (segment (start 145.56525 122.9) (end 145.5955 122.93025) (width 0.2) (layer "B.Cu") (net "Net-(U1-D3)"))
 (segment (start 145.55 122.9) (end 145.56525 122.9) (width 0.2) (layer "B.Cu") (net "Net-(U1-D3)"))
 (segment (start 145.93525 120.73) (end 145.5955 120.39025) (width 0.2) (layer "F.Cu") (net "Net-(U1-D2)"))
 (segment (start 147.883334 120.73) (end 145.93525 120.73) (width 0.2) (layer "F.Cu") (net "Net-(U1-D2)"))
 (via (at 147.883334 120.73) (size 0.6) (drill 0.3) (layers "F.Cu" "B.Cu") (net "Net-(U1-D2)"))
 (via (at 145.5955 120.39025) (size 0.6) (drill 0.3) (layers "F.Cu" "B.Cu") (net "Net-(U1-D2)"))
 (segment (start 125.95 136.33) (end 143.803435 136.33) (width 0.2) (layer "B.Cu") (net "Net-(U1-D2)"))
 (segment (start 148.683334 121.53) (end 147.883334 120.73) (width 0.2) (layer "B.Cu") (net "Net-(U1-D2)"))
 (segment (start 148.683334 138.409899) (end 148.683334 121.53) (width 0.2) (layer "B.Cu") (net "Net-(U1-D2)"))
 (segment (start 146.703435 139.23) (end 147.863233 139.23) (width 0.2) (layer "B.Cu") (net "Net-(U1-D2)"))
 (segment (start 121.91 140.37) (end 125.95 136.33) (width 0.2) (layer "B.Cu") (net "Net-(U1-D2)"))
 (segment (start 147.863233 139.23) (end 148.683334 138.409899) (width 0.2) (layer "B.Cu") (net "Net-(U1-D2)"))
 (segment (start 143.803435 136.33) (end 146.703435 139.23) (width 0.2) (layer "B.Cu") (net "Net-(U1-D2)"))
 (segment (start 158.189611 144.11) (end 159.183723 144.11) (width 0.2) (layer "F.Cu") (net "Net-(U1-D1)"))
 (segment (start 159.183723 144.11) (end 163.663723 139.63) (width 0.2) (layer "F.Cu") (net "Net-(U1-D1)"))
 (segment (start 167.052252 139.63) (end 168.106667 138.575585) (width 0.2) (layer "F.Cu") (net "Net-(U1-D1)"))
 (segment (start 140.933334 140.37) (end 154.449611 140.37) (width 0.2) (layer "F.Cu") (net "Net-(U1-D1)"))
 (segment (start 163.663723 139.63) (end 167.052252 139.63) (width 0.2) (layer "F.Cu") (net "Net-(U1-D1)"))
 (segment (start 163.85025 117.85025) (end 145.5955 117.85025) (width 0.2) (layer "F.Cu") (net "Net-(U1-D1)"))
 (segment (start 154.449611 140.37) (end 158.189611 144.11) (width 0.2) (layer "F.Cu") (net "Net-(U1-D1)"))
 (segment (start 168.106667 122.106667) (end 163.85025 117.85025) (width 0.2) (layer "F.Cu") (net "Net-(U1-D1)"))
 (segment (start 168.106667 138.575585) (end 168.106667 122.106667) (width 0.2) (layer "F.Cu") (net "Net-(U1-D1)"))
 (via (at 145.5955 117.85025) (size 0.6) (drill 0.3) (layers "F.Cu" "B.Cu") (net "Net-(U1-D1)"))
 (segment (start 168.506667 138.741271) (end 167.017938 140.23) (width 0.2) (layer "F.Cu") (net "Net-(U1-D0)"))
 (segment (start 168.506667 121.940982) (end 168.506667 138.741271) (width 0.2) (layer "F.Cu") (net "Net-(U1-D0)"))
 (segment (start 167.017938 140.23) (end 164.18 140.23) (width 0.2) (layer "F.Cu") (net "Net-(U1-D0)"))
 (segment (start 161.945685 115.38) (end 168.506667 121.940982) (width 0.2) (layer "F.Cu") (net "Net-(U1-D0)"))
 (segment (start 145.63 115.38) (end 161.945685 115.38) (width 0.2) (layer "F.Cu") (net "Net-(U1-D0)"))
 (via (at 164.18 140.23) (size 0.6) (drill 0.3) (layers "F.Cu" "B.Cu") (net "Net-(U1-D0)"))
 (via (at 145.63 115.38) (size 0.6) (drill 0.3) (layers "F.Cu" "B.Cu") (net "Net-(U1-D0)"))
 (segment (start 145.5955 115.31025) (end 145.5955 115.3455) (width 0.2) (layer "B.Cu") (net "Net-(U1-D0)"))
 (segment (start 164.18 140.23) (end 164.09 140.23) (width 0.2) (layer "B.Cu") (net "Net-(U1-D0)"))
 (segment (start 145.5955 115.3455) (end 145.63 115.38) (width 0.2) (layer "B.Cu") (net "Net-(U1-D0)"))
 (segment (start 164.09 140.23) (end 163.95 140.37) (width 0.2) (layer "B.Cu") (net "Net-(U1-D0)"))
 (segment (start 163.95 140.37) (end 159.956667 140.37) (width 0.2) (layer "B.Cu") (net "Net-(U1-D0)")))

